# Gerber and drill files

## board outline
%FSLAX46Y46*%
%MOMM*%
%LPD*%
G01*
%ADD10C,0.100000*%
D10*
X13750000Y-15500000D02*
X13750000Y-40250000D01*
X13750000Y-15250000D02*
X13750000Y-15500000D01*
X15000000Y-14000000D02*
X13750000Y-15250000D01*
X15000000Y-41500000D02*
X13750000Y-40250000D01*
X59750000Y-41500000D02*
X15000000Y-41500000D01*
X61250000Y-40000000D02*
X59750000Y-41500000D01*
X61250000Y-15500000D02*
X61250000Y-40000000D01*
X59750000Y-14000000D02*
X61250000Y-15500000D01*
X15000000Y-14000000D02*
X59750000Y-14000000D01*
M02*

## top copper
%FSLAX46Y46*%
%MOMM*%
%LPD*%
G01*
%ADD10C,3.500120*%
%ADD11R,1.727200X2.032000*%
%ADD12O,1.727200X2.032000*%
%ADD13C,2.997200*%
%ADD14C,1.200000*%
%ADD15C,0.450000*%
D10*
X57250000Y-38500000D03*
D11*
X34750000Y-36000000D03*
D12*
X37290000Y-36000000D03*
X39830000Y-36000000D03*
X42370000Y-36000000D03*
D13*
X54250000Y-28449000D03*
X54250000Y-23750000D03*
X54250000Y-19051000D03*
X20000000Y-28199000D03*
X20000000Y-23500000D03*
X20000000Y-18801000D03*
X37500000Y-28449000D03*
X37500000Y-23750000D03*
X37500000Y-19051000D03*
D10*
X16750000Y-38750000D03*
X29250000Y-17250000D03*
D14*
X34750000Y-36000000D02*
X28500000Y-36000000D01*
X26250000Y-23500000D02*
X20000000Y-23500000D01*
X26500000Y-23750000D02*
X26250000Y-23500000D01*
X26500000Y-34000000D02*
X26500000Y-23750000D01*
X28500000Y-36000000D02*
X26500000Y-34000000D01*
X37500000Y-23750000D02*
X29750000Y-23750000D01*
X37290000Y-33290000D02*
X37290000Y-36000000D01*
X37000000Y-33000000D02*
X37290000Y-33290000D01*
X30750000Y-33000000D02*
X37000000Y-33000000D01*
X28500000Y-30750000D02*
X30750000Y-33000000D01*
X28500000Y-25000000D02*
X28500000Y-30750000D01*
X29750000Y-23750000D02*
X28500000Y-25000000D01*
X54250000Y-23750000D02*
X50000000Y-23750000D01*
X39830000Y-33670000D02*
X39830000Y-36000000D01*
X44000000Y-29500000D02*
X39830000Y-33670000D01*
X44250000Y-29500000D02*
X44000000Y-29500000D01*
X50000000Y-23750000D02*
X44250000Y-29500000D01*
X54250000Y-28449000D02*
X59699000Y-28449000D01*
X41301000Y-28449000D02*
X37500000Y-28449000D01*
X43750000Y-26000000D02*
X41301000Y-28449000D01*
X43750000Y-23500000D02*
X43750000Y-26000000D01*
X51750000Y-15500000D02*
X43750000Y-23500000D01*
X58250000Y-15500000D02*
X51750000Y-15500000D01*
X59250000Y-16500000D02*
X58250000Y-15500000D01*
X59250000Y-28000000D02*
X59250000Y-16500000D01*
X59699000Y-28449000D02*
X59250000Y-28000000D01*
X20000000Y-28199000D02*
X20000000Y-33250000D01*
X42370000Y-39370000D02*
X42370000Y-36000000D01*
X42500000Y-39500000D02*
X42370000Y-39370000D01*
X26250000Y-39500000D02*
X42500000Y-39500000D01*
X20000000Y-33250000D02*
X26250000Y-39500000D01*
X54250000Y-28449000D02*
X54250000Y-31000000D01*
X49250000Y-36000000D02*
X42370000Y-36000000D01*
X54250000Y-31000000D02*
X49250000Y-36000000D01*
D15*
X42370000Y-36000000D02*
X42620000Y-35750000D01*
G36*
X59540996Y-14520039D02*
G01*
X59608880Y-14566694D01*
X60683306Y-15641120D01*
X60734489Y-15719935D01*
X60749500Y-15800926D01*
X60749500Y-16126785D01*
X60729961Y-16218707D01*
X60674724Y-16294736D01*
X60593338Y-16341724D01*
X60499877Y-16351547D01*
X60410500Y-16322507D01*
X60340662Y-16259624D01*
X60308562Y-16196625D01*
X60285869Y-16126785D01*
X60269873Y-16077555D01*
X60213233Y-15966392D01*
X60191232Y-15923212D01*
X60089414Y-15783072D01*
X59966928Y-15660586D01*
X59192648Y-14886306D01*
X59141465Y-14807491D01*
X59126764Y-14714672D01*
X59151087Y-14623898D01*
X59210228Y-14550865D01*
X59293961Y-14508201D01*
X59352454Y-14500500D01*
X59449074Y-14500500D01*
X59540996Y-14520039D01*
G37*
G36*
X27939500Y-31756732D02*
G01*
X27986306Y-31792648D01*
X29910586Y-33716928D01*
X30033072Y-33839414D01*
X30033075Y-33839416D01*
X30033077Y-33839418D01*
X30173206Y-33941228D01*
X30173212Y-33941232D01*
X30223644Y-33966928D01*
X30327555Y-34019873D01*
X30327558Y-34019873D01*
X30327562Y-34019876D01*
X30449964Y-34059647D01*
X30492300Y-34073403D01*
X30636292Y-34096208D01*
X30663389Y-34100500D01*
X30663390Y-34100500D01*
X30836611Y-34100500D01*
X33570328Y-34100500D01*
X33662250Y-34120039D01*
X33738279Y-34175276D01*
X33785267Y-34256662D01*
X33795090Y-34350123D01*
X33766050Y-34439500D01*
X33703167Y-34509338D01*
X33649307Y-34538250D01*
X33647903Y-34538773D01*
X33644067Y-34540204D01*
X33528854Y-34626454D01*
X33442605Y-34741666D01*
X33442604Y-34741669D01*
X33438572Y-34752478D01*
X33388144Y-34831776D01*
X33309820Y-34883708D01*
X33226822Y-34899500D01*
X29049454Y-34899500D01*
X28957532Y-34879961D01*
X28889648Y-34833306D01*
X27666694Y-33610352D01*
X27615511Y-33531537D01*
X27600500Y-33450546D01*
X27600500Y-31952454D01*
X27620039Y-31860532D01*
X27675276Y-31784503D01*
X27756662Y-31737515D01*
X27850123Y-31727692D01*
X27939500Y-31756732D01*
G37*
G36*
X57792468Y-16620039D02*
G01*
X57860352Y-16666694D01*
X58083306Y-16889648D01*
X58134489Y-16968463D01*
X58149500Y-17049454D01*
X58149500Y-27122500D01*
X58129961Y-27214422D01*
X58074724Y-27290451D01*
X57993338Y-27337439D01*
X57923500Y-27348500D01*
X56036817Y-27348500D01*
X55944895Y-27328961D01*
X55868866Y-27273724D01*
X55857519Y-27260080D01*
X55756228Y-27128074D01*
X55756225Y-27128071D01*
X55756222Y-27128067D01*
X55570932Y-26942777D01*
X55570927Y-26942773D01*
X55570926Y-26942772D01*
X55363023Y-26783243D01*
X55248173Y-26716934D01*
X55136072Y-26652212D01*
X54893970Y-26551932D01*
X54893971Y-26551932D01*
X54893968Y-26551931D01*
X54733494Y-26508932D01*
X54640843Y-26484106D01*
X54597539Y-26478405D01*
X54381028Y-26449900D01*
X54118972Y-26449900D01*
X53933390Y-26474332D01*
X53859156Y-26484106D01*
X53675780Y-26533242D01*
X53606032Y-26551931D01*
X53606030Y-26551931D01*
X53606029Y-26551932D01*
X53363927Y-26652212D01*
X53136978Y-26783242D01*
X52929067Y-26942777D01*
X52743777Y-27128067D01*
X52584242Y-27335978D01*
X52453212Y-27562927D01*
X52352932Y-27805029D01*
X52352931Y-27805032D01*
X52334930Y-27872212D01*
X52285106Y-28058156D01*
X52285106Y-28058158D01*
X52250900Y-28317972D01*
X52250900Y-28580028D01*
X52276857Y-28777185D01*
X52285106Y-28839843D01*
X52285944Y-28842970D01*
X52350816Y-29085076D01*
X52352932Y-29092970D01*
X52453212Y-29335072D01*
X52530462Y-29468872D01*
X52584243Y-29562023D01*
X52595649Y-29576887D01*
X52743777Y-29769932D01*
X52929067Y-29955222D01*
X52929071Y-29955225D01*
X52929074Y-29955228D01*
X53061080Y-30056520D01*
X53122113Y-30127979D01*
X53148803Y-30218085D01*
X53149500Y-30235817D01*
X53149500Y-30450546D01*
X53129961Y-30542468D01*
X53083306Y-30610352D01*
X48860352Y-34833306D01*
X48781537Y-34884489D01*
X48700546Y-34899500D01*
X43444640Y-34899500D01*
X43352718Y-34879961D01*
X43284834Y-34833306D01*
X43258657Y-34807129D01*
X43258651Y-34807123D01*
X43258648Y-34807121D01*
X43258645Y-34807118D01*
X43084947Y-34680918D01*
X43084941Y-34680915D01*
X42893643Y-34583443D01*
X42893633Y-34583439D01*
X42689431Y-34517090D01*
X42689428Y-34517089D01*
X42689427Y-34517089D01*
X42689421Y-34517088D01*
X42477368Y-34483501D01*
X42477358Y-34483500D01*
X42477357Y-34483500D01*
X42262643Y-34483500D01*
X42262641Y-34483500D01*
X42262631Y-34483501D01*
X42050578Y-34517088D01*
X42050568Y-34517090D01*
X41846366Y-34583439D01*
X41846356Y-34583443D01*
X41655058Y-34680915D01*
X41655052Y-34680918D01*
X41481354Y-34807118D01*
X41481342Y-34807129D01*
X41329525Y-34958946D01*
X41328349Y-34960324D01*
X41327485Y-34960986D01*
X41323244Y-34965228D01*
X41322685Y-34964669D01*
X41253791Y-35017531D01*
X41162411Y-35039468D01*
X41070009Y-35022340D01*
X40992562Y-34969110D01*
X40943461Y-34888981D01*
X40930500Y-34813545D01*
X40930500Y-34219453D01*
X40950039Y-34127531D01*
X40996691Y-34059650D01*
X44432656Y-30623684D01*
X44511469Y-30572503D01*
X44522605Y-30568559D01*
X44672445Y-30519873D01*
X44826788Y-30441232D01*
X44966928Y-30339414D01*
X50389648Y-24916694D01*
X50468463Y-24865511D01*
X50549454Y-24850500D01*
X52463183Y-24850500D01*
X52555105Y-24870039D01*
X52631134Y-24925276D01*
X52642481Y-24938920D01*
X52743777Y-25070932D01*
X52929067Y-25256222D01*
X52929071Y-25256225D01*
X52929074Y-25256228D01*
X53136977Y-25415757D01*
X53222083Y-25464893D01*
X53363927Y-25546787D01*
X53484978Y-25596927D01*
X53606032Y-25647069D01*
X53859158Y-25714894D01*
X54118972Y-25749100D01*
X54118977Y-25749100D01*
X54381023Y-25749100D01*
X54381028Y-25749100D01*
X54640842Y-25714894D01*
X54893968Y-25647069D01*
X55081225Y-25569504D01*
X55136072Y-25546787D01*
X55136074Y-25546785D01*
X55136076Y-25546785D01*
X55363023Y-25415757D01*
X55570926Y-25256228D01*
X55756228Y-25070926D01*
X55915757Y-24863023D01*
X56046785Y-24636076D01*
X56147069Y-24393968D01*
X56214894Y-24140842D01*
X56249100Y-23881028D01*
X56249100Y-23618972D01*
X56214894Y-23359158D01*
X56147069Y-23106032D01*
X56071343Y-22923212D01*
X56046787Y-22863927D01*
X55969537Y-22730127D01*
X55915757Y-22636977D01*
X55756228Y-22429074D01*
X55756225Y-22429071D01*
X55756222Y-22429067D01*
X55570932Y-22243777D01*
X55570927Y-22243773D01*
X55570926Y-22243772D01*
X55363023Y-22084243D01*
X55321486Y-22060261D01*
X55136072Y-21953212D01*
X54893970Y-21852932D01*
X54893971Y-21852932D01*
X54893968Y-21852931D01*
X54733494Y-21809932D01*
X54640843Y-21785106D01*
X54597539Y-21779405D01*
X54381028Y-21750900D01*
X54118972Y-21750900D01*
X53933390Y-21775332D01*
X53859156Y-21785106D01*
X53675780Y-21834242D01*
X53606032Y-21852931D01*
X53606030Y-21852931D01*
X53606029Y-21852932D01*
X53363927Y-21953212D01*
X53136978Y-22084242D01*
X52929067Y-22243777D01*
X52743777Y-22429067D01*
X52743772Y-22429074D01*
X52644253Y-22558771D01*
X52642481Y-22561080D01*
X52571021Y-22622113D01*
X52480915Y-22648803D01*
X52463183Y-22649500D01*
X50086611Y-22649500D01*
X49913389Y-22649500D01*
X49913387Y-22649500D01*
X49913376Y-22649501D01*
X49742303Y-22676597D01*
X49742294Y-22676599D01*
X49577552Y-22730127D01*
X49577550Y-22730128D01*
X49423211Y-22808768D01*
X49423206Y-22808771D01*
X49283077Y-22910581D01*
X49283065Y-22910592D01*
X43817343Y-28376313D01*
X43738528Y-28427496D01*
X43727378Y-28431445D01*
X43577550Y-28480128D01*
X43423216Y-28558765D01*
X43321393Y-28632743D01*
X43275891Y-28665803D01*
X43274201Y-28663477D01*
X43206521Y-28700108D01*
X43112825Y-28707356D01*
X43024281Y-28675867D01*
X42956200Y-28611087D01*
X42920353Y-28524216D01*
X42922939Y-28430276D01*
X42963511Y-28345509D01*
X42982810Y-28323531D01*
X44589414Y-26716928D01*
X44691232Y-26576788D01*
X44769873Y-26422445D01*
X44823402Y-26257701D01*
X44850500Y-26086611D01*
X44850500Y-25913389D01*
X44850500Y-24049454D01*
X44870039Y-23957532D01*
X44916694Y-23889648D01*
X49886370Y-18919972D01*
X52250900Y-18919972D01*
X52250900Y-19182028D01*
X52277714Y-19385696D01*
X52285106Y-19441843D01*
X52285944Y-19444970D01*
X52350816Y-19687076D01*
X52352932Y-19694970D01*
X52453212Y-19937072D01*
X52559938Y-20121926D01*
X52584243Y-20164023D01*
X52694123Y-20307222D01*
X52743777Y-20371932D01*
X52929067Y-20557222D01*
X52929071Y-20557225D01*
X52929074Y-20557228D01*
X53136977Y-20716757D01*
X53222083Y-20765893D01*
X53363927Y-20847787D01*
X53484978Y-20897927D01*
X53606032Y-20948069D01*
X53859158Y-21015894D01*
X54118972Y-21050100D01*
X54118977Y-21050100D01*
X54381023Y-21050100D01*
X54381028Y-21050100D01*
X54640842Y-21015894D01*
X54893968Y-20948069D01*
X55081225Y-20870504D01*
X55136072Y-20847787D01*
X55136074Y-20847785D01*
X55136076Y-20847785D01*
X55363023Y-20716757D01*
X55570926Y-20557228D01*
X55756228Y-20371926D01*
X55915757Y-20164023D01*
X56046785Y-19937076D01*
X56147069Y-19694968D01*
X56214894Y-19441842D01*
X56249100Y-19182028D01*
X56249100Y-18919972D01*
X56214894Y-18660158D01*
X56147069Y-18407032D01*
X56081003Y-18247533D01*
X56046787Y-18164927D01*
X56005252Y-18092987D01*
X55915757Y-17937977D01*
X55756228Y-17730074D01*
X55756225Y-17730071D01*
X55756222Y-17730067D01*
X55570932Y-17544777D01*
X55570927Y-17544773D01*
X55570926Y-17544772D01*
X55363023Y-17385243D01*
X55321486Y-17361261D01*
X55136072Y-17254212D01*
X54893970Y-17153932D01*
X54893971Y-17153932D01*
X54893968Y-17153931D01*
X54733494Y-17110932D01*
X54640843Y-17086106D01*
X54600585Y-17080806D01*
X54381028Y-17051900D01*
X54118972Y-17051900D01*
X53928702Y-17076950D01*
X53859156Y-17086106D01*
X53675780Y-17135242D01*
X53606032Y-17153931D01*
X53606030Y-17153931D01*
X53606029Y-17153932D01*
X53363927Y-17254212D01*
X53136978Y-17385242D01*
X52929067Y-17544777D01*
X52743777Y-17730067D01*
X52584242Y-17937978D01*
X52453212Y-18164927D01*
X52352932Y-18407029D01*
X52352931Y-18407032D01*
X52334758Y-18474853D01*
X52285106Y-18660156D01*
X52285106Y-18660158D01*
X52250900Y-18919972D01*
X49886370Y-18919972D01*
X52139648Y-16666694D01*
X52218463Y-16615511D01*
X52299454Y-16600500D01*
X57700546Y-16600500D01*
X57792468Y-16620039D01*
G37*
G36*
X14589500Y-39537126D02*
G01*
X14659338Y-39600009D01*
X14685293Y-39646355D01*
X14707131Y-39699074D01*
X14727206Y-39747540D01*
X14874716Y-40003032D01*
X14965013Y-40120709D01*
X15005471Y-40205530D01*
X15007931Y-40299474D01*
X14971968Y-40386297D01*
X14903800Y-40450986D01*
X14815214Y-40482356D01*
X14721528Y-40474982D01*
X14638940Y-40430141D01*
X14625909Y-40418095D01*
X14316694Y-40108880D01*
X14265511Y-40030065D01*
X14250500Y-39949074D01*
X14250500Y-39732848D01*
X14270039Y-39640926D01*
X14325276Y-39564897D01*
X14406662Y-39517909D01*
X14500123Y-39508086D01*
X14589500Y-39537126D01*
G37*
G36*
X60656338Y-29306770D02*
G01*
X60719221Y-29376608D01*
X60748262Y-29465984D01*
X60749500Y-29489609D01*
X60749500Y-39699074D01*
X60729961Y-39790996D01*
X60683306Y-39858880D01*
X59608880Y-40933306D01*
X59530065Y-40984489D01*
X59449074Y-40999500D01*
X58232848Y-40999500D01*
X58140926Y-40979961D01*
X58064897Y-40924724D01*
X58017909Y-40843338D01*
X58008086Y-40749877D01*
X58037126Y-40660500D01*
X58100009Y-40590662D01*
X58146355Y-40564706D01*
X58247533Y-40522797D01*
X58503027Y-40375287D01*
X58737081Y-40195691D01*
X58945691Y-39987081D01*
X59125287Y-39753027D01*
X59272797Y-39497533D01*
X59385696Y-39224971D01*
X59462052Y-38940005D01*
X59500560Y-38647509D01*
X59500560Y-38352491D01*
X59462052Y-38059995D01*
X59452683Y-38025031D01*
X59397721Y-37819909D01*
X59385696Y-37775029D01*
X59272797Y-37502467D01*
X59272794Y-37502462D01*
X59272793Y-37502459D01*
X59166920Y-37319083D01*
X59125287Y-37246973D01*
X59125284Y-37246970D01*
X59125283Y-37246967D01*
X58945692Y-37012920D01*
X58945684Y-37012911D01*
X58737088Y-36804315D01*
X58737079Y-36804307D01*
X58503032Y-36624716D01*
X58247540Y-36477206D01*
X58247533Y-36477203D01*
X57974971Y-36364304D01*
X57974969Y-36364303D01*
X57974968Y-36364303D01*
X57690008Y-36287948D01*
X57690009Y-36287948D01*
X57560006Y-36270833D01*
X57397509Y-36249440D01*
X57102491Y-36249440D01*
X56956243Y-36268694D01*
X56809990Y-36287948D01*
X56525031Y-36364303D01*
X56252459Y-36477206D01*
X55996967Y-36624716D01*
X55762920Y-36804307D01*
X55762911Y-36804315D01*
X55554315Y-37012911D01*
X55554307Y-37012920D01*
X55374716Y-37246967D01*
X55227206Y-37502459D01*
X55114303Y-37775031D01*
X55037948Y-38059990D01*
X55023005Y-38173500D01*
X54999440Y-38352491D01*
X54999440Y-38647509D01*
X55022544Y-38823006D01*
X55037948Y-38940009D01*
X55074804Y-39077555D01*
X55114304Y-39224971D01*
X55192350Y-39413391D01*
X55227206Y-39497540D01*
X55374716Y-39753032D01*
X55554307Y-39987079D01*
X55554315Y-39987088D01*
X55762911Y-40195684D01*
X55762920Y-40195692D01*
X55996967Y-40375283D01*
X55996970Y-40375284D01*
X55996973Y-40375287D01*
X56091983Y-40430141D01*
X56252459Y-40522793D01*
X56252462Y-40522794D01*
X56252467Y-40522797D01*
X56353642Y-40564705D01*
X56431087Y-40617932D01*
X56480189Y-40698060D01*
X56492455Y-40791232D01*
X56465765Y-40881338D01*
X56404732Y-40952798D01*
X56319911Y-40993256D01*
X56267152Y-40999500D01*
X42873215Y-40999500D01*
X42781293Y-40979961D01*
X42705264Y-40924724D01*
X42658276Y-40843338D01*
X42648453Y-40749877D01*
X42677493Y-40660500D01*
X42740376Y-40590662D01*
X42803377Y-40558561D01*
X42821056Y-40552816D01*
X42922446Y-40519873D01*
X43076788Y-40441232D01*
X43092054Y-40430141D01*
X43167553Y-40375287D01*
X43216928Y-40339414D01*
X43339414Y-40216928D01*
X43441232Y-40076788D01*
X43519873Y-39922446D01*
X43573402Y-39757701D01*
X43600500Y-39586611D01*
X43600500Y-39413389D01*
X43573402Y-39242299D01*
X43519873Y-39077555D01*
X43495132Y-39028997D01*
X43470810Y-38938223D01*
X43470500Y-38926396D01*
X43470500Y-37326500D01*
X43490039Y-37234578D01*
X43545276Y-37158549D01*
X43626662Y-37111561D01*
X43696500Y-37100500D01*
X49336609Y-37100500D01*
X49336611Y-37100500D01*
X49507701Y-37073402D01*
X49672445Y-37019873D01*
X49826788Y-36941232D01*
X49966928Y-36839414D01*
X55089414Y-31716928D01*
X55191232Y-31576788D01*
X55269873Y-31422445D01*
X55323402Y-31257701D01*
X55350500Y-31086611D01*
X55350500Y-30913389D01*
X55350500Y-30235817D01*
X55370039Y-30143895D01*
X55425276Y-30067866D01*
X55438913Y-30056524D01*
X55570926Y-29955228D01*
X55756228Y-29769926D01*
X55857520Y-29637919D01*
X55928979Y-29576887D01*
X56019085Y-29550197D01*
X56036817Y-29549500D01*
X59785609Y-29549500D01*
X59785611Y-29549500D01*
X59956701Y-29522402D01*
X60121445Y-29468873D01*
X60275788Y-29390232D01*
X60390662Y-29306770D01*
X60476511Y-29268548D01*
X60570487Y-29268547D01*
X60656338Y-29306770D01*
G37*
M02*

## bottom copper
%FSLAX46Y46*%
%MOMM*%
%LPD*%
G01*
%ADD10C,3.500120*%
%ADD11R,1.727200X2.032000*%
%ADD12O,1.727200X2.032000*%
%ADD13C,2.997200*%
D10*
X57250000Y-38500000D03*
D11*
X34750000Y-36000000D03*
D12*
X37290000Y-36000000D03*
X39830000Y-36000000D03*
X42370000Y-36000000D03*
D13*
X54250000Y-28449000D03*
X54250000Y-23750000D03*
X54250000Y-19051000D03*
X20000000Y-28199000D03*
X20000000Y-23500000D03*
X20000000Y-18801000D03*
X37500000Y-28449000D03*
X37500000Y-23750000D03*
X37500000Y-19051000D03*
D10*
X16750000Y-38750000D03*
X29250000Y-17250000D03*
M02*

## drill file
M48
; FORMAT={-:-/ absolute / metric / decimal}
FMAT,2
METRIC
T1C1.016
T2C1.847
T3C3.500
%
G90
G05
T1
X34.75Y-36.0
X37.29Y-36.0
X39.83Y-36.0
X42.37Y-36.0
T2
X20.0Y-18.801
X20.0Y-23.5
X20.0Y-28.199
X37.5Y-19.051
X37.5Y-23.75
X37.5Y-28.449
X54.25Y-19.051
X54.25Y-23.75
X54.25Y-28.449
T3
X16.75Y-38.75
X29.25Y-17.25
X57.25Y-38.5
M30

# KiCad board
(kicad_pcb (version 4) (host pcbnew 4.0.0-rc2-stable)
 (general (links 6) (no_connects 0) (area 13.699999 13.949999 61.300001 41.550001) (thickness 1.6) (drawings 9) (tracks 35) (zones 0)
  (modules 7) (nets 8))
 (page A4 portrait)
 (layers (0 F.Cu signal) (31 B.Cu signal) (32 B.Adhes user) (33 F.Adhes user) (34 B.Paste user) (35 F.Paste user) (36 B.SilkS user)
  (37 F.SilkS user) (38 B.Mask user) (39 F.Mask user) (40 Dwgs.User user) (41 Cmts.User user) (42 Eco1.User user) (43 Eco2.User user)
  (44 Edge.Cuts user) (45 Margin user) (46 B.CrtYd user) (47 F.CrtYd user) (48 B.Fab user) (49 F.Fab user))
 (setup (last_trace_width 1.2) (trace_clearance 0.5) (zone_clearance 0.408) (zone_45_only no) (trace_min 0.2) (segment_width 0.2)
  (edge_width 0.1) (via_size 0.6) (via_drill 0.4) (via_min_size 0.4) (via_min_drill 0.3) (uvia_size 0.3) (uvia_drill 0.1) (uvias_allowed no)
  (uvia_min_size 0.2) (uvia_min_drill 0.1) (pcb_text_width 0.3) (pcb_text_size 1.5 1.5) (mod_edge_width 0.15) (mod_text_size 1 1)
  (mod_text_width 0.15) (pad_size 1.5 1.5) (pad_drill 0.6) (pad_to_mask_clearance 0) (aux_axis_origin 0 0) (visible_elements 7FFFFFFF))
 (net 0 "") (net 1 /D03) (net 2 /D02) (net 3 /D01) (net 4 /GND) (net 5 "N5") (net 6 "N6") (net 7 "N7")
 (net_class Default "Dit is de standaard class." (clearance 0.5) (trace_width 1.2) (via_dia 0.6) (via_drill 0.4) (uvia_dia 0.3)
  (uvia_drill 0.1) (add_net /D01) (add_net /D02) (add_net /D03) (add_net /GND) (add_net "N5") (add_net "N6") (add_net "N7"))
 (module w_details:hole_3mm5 (layer F.Cu) (at 57.25 38.5)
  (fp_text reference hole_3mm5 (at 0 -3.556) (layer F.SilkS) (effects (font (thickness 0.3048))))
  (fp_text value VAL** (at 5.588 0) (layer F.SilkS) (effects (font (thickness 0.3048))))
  (pad 1 thru_hole circle (at 0 0) (size 3.50012 3.50012) (drill 3.50012) (layers *.Cu F.SilkS)))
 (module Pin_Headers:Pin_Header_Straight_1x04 (layer F.Cu) (at 34.75 36 90)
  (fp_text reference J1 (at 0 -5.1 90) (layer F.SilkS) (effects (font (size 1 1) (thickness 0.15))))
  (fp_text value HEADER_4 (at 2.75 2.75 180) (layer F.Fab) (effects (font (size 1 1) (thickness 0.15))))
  (pad 1 thru_hole rect (at 0 0 90) (size 2.032 1.7272) (drill 1.016) (layers *.Cu *.Mask F.SilkS) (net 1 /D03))
  (pad 2 thru_hole oval (at 0 2.54 90) (size 2.032 1.7272) (drill 1.016) (layers *.Cu *.Mask F.SilkS) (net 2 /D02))
  (pad 3 thru_hole oval (at 0 5.08 90) (size 2.032 1.7272) (drill 1.016) (layers *.Cu *.Mask F.SilkS) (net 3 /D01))
  (pad 4 thru_hole oval (at 0 7.62 90) (size 2.032 1.7272) (drill 1.016) (layers *.Cu *.Mask F.SilkS) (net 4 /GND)))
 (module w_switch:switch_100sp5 (layer F.Cu) (at 54.25 23.75 90)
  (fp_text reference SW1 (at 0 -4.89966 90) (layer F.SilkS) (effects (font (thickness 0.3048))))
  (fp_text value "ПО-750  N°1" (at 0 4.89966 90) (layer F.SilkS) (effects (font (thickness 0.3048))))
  (pad 1 thru_hole circle (at -4.699 0 90) (size 2.9972 2.9972) (drill 1.84658) (layers *.Cu *.Mask F.SilkS) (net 4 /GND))
  (pad 2 thru_hole circle (at 0 0 90) (size 2.9972 2.9972) (drill 1.84658) (layers *.Cu *.Mask F.SilkS) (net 3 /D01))
  (pad 3 thru_hole circle (at 4.699 0 90) (size 2.9972 2.9972) (drill 1.84658) (layers *.Cu *.Mask F.SilkS) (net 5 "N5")))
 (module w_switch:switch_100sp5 (layer F.Cu) (at 20 23.5 90)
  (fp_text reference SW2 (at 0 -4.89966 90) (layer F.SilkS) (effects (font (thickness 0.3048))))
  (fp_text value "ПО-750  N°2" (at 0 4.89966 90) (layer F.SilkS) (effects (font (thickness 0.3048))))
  (pad 1 thru_hole circle (at -4.699 0 90) (size 2.9972 2.9972) (drill 1.84658) (layers *.Cu *.Mask F.SilkS) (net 4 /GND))
  (pad 2 thru_hole circle (at 0 0 90) (size 2.9972 2.9972) (drill 1.84658) (layers *.Cu *.Mask F.SilkS) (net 1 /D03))
  (pad 3 thru_hole circle (at 4.699 0 90) (size 2.9972 2.9972) (drill 1.84658) (layers *.Cu *.Mask F.SilkS) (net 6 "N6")))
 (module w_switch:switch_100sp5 (layer F.Cu) (at 37.5 23.75 90)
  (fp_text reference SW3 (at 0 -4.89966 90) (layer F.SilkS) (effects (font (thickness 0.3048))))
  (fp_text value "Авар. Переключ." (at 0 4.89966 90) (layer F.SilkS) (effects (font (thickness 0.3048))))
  (pad 1 thru_hole circle (at -4.699 0 90) (size 2.9972 2.9972) (drill 1.84658) (layers *.Cu *.Mask F.SilkS) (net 4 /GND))
  (pad 2 thru_hole circle (at 0 0 90) (size 2.9972 2.9972) (drill 1.84658) (layers *.Cu *.Mask F.SilkS) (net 2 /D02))
  (pad 3 thru_hole circle (at 4.699 0 90) (size 2.9972 2.9972) (drill 1.84658) (layers *.Cu *.Mask F.SilkS) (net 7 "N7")))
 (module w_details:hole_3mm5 (layer F.Cu) (at 16.75 38.75)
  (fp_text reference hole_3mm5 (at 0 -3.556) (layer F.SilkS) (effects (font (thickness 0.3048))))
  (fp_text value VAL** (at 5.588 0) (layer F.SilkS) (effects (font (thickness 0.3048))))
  (pad 1 thru_hole circle (at 0 0) (size 3.50012 3.50012) (drill 3.50012) (layers *.Cu F.SilkS)))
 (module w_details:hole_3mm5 (layer F.Cu) (at 29.25 17.25)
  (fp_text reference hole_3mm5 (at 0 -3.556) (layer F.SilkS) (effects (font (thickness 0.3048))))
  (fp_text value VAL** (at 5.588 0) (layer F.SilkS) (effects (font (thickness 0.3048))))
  (pad 1 thru_hole circle (at 0 0) (size 3.50012 3.50012) (drill 3.50012) (layers *.Cu F.SilkS)))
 (gr_line (start 13.75 15.5) (end 13.75 40.25) (angle 90) (layer Edge.Cuts) (width 0.1))
 (gr_line (start 13.75 15.25) (end 13.75 15.5) (angle 90) (layer Edge.Cuts) (width 0.1))
 (gr_line (start 15 14) (end 13.75 15.25) (angle 90) (layer Edge.Cuts) (width 0.1))
 (gr_line (start 15 41.5) (end 13.75 40.25) (angle 90) (layer Edge.Cuts) (width 0.1))
 (gr_line (start 59.75 41.5) (end 15 41.5) (angle 90) (layer Edge.Cuts) (width 0.1))
 (gr_line (start 61.25 40) (end 59.75 41.5) (angle 90) (layer Edge.Cuts) (width 0.1))
 (gr_line (start 61.25 15.5) (end 61.25 40) (angle 90) (layer Edge.Cuts) (width 0.1))
 (gr_line (start 59.75 14) (end 61.25 15.5) (angle 90) (layer Edge.Cuts) (width 0.1))
 (gr_line (start 15 14) (end 59.75 14) (angle 90) (layer Edge.Cuts) (width 0.1))
 (segment (start 34.75 36) (end 28.5 36) (width 1.2) (layer F.Cu) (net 1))
 (segment (start 26.25 23.5) (end 20 23.5) (width 1.2) (layer F.Cu) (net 1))
 (segment (start 26.5 23.75) (end 26.25 23.5) (width 1.2) (layer F.Cu) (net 1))
 (segment (start 26.5 34) (end 26.5 23.75) (width 1.2) (layer F.Cu) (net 1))
 (segment (start 28.5 36) (end 26.5 34) (width 1.2) (layer F.Cu) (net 1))
 (segment (start 37.5 23.75) (end 29.75 23.75) (width 1.2) (layer F.Cu) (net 2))
 (segment (start 37.29 33.29) (end 37.29 36) (width 1.2) (layer F.Cu) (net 2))
 (segment (start 37 33) (end 37.29 33.29) (width 1.2) (layer F.Cu) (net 2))
 (segment (start 30.75 33) (end 37 33) (width 1.2) (layer F.Cu) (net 2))
 (segment (start 28.5 30.75) (end 30.75 33) (width 1.2) (layer F.Cu) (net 2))
 (segment (start 28.5 25) (end 28.5 30.75) (width 1.2) (layer F.Cu) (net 2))
 (segment (start 29.75 23.75) (end 28.5 25) (width 1.2) (layer F.Cu) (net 2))
 (segment (start 54.25 23.75) (end 50 23.75) (width 1.2) (layer F.Cu) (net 3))
 (segment (start 39.83 33.67) (end 39.83 36) (width 1.2) (layer F.Cu) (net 3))
 (segment (start 44 29.5) (end 39.83 33.67) (width 1.2) (layer F.Cu) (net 3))
 (segment (start 44.25 29.5) (end 44 29.5) (width 1.2) (layer F.Cu) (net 3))
 (segment (start 50 23.75) (end 44.25 29.5) (width 1.2) (layer F.Cu) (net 3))
 (segment (start 54.25 28.449) (end 59.699 28.449) (width 1.2) (layer F.Cu) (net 4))
 (segment (start 41.301 28.449) (end 37.5 28.449) (width 1.2) (layer F.Cu) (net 4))
 (segment (start 43.75 26) (end 41.301 28.449) (width 1.2) (layer F.Cu) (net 4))
 (segment (start 43.75 23.5) (end 43.75 26) (width 1.2) (layer F.Cu) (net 4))
 (segment (start 51.75 15.5) (end 43.75 23.5) (width 1.2) (layer F.Cu) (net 4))
 (segment (start 58.25 15.5) (end 51.75 15.5) (width 1.2) (layer F.Cu) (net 4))
 (segment (start 59.25 16.5) (end 58.25 15.5) (width 1.2) (layer F.Cu) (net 4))
 (segment (start 59.25 28) (end 59.25 16.5) (width 1.2) (layer F.Cu) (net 4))
 (segment (start 59.699 28.449) (end 59.25 28) (width 1.2) (layer F.Cu) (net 4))
 (segment (start 20 28.199) (end 20 33.25) (width 1.2) (layer F.Cu) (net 4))
 (segment (start 42.37 39.37) (end 42.37 36) (width 1.2) (layer F.Cu) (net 4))
 (segment (start 42.5 39.5) (end 42.37 39.37) (width 1.2) (layer F.Cu) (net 4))
 (segment (start 26.25 39.5) (end 42.5 39.5) (width 1.2) (layer F.Cu) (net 4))
 (segment (start 20 33.25) (end 26.25 39.5) (width 1.2) (layer F.Cu) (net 4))
 (segment (start 54.25 28.449) (end 54.25 31) (width 1.2) (layer F.Cu) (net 4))
 (segment (start 49.25 36) (end 42.37 36) (width 1.2) (layer F.Cu) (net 4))
 (segment (start 54.25 31) (end 49.25 36) (width 1.2) (layer F.Cu) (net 4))
 (segment (start 42.37 36) (end 42.62 35.75) (width 0.45) (layer F.Cu) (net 4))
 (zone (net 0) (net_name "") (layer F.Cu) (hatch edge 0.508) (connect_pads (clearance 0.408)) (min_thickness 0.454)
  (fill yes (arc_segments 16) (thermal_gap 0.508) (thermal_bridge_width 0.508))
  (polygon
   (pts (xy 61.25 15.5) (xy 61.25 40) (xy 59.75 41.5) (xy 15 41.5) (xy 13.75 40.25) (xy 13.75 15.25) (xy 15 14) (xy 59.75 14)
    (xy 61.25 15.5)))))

